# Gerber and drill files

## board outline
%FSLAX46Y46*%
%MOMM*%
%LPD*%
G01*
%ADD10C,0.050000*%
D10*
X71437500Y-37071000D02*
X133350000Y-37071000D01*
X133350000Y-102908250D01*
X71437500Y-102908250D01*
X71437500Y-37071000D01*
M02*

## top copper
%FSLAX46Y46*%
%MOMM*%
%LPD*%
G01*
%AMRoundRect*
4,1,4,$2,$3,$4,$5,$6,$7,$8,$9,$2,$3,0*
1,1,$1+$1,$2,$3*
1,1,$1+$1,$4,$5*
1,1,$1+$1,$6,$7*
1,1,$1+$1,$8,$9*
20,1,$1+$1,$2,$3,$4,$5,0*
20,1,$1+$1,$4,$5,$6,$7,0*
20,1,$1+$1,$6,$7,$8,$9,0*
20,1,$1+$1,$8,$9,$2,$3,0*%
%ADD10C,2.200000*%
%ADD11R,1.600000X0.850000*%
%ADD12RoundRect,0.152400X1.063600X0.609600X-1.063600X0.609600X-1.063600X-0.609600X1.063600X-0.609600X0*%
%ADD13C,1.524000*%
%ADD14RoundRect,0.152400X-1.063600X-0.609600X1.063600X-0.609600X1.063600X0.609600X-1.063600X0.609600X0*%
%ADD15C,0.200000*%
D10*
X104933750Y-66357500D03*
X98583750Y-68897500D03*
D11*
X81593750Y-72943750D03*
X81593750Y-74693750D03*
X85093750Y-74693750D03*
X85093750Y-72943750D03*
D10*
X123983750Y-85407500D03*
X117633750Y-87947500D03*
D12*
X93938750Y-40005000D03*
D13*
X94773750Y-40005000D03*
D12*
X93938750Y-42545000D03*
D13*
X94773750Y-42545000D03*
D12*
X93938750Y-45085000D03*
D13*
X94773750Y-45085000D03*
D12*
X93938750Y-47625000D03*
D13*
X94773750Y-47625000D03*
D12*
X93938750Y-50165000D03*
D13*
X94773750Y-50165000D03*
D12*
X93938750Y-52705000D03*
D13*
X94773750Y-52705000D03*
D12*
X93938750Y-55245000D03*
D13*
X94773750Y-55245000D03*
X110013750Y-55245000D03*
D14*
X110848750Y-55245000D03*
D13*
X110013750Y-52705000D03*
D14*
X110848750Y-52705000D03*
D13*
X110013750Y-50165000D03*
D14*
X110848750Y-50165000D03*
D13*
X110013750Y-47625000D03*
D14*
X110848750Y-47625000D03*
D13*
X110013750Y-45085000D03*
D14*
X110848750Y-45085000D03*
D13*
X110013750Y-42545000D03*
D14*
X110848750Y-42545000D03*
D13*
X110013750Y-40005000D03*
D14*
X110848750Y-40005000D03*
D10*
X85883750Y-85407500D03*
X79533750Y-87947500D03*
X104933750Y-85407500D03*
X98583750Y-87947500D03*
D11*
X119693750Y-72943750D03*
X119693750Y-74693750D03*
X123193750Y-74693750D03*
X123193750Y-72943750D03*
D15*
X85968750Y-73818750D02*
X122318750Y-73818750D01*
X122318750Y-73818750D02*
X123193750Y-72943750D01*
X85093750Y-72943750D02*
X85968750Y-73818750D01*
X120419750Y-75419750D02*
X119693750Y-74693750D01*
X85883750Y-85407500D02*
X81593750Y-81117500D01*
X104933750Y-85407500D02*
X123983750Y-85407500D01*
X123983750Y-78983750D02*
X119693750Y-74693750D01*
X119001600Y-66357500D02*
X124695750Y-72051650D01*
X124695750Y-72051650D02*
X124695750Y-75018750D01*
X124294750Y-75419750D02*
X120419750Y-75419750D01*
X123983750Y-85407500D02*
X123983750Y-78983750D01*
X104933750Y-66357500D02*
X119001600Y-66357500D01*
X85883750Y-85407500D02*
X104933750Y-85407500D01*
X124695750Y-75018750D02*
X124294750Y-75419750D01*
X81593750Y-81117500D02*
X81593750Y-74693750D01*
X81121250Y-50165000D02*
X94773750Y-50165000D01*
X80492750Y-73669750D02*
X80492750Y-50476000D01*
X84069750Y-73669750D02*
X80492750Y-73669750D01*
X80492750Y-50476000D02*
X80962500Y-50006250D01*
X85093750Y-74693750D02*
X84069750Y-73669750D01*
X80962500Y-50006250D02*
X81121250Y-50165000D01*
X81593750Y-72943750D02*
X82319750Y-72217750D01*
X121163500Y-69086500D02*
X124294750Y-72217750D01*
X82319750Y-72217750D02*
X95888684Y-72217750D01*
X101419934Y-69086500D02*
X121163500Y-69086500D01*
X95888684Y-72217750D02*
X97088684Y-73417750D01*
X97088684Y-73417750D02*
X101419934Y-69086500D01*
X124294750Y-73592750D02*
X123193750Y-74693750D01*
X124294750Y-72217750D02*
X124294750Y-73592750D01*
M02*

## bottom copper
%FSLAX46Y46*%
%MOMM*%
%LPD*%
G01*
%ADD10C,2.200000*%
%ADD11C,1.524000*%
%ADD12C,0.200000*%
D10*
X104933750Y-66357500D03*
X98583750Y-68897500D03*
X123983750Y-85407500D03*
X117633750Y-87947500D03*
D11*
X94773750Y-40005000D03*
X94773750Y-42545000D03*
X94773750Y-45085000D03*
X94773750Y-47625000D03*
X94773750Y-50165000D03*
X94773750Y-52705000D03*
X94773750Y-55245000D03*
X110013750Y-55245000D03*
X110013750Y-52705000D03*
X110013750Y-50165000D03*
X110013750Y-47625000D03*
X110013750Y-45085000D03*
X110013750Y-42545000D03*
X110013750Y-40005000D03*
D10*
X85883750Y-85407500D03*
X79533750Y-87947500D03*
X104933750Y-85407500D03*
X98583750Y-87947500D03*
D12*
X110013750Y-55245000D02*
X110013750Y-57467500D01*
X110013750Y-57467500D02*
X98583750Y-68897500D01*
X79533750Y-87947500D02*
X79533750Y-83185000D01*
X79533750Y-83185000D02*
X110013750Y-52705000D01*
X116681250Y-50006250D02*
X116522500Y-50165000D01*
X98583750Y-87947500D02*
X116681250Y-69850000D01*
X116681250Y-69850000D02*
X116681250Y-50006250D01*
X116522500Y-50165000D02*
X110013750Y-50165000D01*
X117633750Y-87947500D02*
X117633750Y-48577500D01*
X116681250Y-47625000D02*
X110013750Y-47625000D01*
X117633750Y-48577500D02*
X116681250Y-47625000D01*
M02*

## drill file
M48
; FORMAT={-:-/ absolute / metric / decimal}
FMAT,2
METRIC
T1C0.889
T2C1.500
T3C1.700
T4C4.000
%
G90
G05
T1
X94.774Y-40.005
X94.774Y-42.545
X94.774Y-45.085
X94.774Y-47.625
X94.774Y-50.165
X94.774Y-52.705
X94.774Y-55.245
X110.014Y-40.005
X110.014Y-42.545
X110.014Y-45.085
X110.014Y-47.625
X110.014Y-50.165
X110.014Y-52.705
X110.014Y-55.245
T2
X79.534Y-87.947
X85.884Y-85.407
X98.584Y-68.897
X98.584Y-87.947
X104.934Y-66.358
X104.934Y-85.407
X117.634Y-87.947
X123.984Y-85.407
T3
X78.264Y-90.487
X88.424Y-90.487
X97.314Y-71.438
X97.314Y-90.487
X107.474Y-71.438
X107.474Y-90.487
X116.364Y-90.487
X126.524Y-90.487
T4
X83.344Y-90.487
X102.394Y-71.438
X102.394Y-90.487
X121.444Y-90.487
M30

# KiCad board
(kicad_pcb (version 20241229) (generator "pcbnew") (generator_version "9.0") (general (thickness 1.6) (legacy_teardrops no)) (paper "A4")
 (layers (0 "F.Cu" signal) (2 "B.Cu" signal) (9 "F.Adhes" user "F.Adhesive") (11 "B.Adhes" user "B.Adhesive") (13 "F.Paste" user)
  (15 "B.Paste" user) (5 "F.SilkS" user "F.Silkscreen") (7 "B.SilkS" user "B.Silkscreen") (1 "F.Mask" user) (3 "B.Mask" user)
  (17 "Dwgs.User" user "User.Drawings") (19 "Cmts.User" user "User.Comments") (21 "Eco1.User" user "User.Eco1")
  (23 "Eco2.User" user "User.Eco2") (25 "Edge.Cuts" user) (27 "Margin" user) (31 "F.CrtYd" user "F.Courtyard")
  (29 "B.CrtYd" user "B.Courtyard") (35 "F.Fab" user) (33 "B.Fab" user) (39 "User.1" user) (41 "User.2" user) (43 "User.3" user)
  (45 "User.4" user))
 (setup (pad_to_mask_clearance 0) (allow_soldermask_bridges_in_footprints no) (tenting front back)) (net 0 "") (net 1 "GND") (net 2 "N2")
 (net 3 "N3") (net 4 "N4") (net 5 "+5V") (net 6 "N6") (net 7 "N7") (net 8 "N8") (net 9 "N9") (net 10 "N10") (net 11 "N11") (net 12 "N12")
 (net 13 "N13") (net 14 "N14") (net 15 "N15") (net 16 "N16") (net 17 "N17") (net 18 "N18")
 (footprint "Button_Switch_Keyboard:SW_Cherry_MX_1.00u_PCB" (layer "F.Cu") (at 104.93375 66.3575)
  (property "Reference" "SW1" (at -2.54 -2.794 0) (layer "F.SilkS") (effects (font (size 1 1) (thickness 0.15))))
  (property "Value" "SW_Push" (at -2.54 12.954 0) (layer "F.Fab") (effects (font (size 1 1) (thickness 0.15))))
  (pad "" np_thru_hole circle (at -7.62 5.08) (size 1.7 1.7) (drill 1.7) (layers "*.Cu" "*.Mask"))
  (pad "" np_thru_hole circle (at -2.54 5.08) (size 4 4) (drill 4) (layers "*.Cu" "*.Mask"))
  (pad "" np_thru_hole circle (at 2.54 5.08) (size 1.7 1.7) (drill 1.7) (layers "*.Cu" "*.Mask"))
  (pad "1" thru_hole circle (at 0 0) (size 2.2 2.2) (drill 1.5) (layers "*.Cu" "*.Mask") (remove_unused_layers no) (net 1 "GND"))
  (pad "2" thru_hole circle (at -6.35 2.54) (size 2.2 2.2) (drill 1.5) (layers "*.Cu" "*.Mask") (remove_unused_layers no) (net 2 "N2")))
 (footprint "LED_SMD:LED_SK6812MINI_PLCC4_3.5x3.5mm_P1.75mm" (layer "F.Cu") (at 83.34375 73.81875)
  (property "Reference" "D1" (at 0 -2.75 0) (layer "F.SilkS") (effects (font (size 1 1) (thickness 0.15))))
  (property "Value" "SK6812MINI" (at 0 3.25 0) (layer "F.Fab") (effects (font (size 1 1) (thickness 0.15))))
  (pad "1" smd rect (at -1.75 -0.875) (size 1.6 0.85) (layers "F.Cu" "F.Mask" "F.Paste") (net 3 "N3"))
  (pad "2" smd rect (at -1.75 0.875) (size 1.6 0.85) (layers "F.Cu" "F.Mask" "F.Paste") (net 1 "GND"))
  (pad "3" smd rect (at 1.75 0.875) (size 1.6 0.85) (layers "F.Cu" "F.Mask" "F.Paste") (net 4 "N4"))
  (pad "4" smd rect (at 1.75 -0.875) (size 1.6 0.85) (layers "F.Cu" "F.Mask" "F.Paste") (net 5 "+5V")))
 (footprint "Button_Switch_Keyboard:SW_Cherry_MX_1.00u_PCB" (layer "F.Cu") (at 123.98375 85.4075)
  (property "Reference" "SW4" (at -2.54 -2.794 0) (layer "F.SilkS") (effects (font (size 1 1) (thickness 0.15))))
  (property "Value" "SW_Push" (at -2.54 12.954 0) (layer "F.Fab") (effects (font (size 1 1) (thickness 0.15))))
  (pad "" np_thru_hole circle (at -7.62 5.08) (size 1.7 1.7) (drill 1.7) (layers "*.Cu" "*.Mask"))
  (pad "" np_thru_hole circle (at -2.54 5.08) (size 4 4) (drill 4) (layers "*.Cu" "*.Mask"))
  (pad "" np_thru_hole circle (at 2.54 5.08) (size 1.7 1.7) (drill 1.7) (layers "*.Cu" "*.Mask"))
  (pad "1" thru_hole circle (at 0 0) (size 2.2 2.2) (drill 1.5) (layers "*.Cu" "*.Mask") (remove_unused_layers no) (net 1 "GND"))
  (pad "2" thru_hole circle (at -6.35 2.54) (size 2.2 2.2) (drill 1.5) (layers "*.Cu" "*.Mask") (remove_unused_layers no) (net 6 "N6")))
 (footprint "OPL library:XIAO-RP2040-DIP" (layer "F.Cu") (at 102.39375 47.625)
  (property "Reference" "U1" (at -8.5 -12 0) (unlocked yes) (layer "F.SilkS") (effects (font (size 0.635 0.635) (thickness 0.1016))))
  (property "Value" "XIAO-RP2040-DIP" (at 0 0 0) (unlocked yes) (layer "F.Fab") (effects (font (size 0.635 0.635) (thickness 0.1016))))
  (pad "1" smd roundrect (at -8.455 -7.62 180) (size 2.432 1.524) (layers "F.Cu" "F.Mask") (roundrect_rratio 0.1) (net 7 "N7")
   (thermal_bridge_angle 45))
  (pad "1" thru_hole circle (at -7.62 -7.62 180) (size 1.524 1.524) (drill 0.889) (layers "*.Cu" "*.Mask") (remove_unused_layers no)
   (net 7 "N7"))
  (pad "2" smd roundrect (at -8.455 -5.08 180) (size 2.432 1.524) (layers "F.Cu" "F.Mask") (roundrect_rratio 0.1) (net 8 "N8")
   (thermal_bridge_angle 45))
  (pad "2" thru_hole circle (at -7.62 -5.08 180) (size 1.524 1.524) (drill 0.889) (layers "*.Cu" "*.Mask") (remove_unused_layers no)
   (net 8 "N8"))
  (pad "3" smd roundrect (at -8.455 -2.54 180) (size 2.432 1.524) (layers "F.Cu" "F.Mask") (roundrect_rratio 0.1) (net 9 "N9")
   (thermal_bridge_angle 45))
  (pad "3" thru_hole circle (at -7.62 -2.54 180) (size 1.524 1.524) (drill 0.889) (layers "*.Cu" "*.Mask") (remove_unused_layers no)
   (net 9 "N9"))
  (pad "4" smd roundrect (at -8.455 0 180) (size 2.432 1.524) (layers "F.Cu" "F.Mask") (roundrect_rratio 0.1) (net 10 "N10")
   (thermal_bridge_angle 45))
  (pad "4" thru_hole circle (at -7.62 0 180) (size 1.524 1.524) (drill 0.889) (layers "*.Cu" "*.Mask") (remove_unused_layers no)
   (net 10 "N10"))
  (pad "5" smd roundrect (at -8.455 2.54 180) (size 2.432 1.524) (layers "F.Cu" "F.Mask") (roundrect_rratio 0.1) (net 4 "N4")
   (thermal_bridge_angle 45))
  (pad "5" thru_hole circle (at -7.62 2.54 180) (size 1.524 1.524) (drill 0.889) (layers "*.Cu" "*.Mask") (remove_unused_layers no)
   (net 4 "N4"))
  (pad "6" smd roundrect (at -8.455 5.08 180) (size 2.432 1.524) (layers "F.Cu" "F.Mask") (roundrect_rratio 0.1) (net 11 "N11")
   (thermal_bridge_angle 45))
  (pad "6" thru_hole circle (at -7.62 5.08 180) (size 1.524 1.524) (drill 0.889) (layers "*.Cu" "*.Mask") (remove_unused_layers no)
   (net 11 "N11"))
  (pad "7" smd roundrect (at -8.455 7.62 180) (size 2.432 1.524) (layers "F.Cu" "F.Mask") (roundrect_rratio 0.1) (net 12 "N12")
   (thermal_bridge_angle 45))
  (pad "7" thru_hole circle (at -7.62 7.62 180) (size 1.524 1.524) (drill 0.889) (layers "*.Cu" "*.Mask") (remove_unused_layers no)
   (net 12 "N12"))
  (pad "8" thru_hole circle (at 7.62 7.62) (size 1.524 1.524) (drill 0.889) (layers "*.Cu" "*.Mask") (remove_unused_layers no) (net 2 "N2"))
  (pad "8" smd roundrect (at 8.455 7.62) (size 2.432 1.524) (layers "F.Cu" "F.Mask") (roundrect_rratio 0.1) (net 2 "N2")
   (thermal_bridge_angle 45))
  (pad "9" thru_hole circle (at 7.62 5.08) (size 1.524 1.524) (drill 0.889) (layers "*.Cu" "*.Mask") (remove_unused_layers no)
   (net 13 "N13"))
  (pad "9" smd roundrect (at 8.455 5.08) (size 2.432 1.524) (layers "F.Cu" "F.Mask") (roundrect_rratio 0.1) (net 13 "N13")
   (thermal_bridge_angle 45))
  (pad "10" thru_hole circle (at 7.62 2.54) (size 1.524 1.524) (drill 0.889) (layers "*.Cu" "*.Mask") (remove_unused_layers no)
   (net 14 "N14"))
  (pad "10" smd roundrect (at 8.455 2.54) (size 2.432 1.524) (layers "F.Cu" "F.Mask") (roundrect_rratio 0.1) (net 14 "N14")
   (thermal_bridge_angle 45))
  (pad "11" thru_hole circle (at 7.62 0) (size 1.524 1.524) (drill 0.889) (layers "*.Cu" "*.Mask") (remove_unused_layers no) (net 6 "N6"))
  (pad "11" smd roundrect (at 8.455 0) (size 2.432 1.524) (layers "F.Cu" "F.Mask") (roundrect_rratio 0.1) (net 6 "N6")
   (thermal_bridge_angle 45))
  (pad "12" thru_hole circle (at 7.62 -2.54) (size 1.524 1.524) (drill 0.889) (layers "*.Cu" "*.Mask") (remove_unused_layers no)
   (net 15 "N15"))
  (pad "12" smd roundrect (at 8.455 -2.54) (size 2.432 1.524) (layers "F.Cu" "F.Mask") (roundrect_rratio 0.1) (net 15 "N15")
   (thermal_bridge_angle 45))
  (pad "13" thru_hole circle (at 7.62 -5.08) (size 1.524 1.524) (drill 0.889) (layers "*.Cu" "*.Mask") (remove_unused_layers no)
   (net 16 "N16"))
  (pad "13" smd roundrect (at 8.455 -5.08) (size 2.432 1.524) (layers "F.Cu" "F.Mask") (roundrect_rratio 0.1) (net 16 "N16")
   (thermal_bridge_angle 45))
  (pad "14" thru_hole circle (at 7.62 -7.62) (size 1.524 1.524) (drill 0.889) (layers "*.Cu" "*.Mask") (remove_unused_layers no)
   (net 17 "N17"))
  (pad "14" smd roundrect (at 8.455 -7.62) (size 2.432 1.524) (layers "F.Cu" "F.Mask") (roundrect_rratio 0.1) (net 17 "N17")
   (thermal_bridge_angle 45)))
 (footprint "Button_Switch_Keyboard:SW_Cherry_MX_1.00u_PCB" (layer "F.Cu") (at 85.88375 85.4075)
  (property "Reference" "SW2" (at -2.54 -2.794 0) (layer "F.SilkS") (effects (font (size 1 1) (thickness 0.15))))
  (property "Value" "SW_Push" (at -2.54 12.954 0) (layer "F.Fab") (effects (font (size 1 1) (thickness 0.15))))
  (pad "" np_thru_hole circle (at -7.62 5.08) (size 1.7 1.7) (drill 1.7) (layers "*.Cu" "*.Mask"))
  (pad "" np_thru_hole circle (at -2.54 5.08) (size 4 4) (drill 4) (layers "*.Cu" "*.Mask"))
  (pad "" np_thru_hole circle (at 2.54 5.08) (size 1.7 1.7) (drill 1.7) (layers "*.Cu" "*.Mask"))
  (pad "1" thru_hole circle (at 0 0) (size 2.2 2.2) (drill 1.5) (layers "*.Cu" "*.Mask") (remove_unused_layers no) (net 1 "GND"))
  (pad "2" thru_hole circle (at -6.35 2.54) (size 2.2 2.2) (drill 1.5) (layers "*.Cu" "*.Mask") (remove_unused_layers no) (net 13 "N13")))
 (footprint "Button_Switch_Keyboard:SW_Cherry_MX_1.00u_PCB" (layer "F.Cu") (at 104.93375 85.4075)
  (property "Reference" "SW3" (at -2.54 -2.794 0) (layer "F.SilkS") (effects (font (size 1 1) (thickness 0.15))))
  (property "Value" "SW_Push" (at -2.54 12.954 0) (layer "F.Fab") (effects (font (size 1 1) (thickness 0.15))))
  (pad "" np_thru_hole circle (at -7.62 5.08) (size 1.7 1.7) (drill 1.7) (layers "*.Cu" "*.Mask"))
  (pad "" np_thru_hole circle (at -2.54 5.08) (size 4 4) (drill 4) (layers "*.Cu" "*.Mask"))
  (pad "" np_thru_hole circle (at 2.54 5.08) (size 1.7 1.7) (drill 1.7) (layers "*.Cu" "*.Mask"))
  (pad "1" thru_hole circle (at 0 0) (size 2.2 2.2) (drill 1.5) (layers "*.Cu" "*.Mask") (remove_unused_layers no) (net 1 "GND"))
  (pad "2" thru_hole circle (at -6.35 2.54) (size 2.2 2.2) (drill 1.5) (layers "*.Cu" "*.Mask") (remove_unused_layers no) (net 14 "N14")))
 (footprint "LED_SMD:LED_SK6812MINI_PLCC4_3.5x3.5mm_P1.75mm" (layer "F.Cu") (at 121.44375 73.81875)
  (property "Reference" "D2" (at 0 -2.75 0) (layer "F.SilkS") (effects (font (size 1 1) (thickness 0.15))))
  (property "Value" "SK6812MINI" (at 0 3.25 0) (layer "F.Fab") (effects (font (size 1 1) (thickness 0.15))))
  (pad "1" smd rect (at -1.75 -0.875) (size 1.6 0.85) (layers "F.Cu" "F.Mask" "F.Paste") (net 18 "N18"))
  (pad "2" smd rect (at -1.75 0.875) (size 1.6 0.85) (layers "F.Cu" "F.Mask" "F.Paste") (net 1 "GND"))
  (pad "3" smd rect (at 1.75 0.875) (size 1.6 0.85) (layers "F.Cu" "F.Mask" "F.Paste") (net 3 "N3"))
  (pad "4" smd rect (at 1.75 -0.875) (size 1.6 0.85) (layers "F.Cu" "F.Mask" "F.Paste") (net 5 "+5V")))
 (gr_rect (start 71.4375 37.071) (end 133.35 102.90825) (stroke (width 0.05) (type default)) (fill no) (layer "Edge.Cuts"))
 (segment (start 85.96875 73.81875) (end 122.31875 73.81875) (width 0.2) (layer "F.Cu") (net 5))
 (segment (start 122.31875 73.81875) (end 123.19375 72.94375) (width 0.2) (layer "F.Cu") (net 5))
 (segment (start 85.09375 72.94375) (end 85.96875 73.81875) (width 0.2) (layer "F.Cu") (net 5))
 (segment (start 120.41975 75.41975) (end 119.69375 74.69375) (width 0.2) (layer "F.Cu") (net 1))
 (segment (start 85.88375 85.4075) (end 81.59375 81.1175) (width 0.2) (layer "F.Cu") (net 1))
 (segment (start 104.93375 85.4075) (end 123.98375 85.4075) (width 0.2) (layer "F.Cu") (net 1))
 (segment (start 123.98375 78.98375) (end 119.69375 74.69375) (width 0.2) (layer "F.Cu") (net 1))
 (segment (start 119.0016 66.3575) (end 124.69575 72.05165) (width 0.2) (layer "F.Cu") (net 1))
 (segment (start 124.69575 72.05165) (end 124.69575 75.01875) (width 0.2) (layer "F.Cu") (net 1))
 (segment (start 124.29475 75.41975) (end 120.41975 75.41975) (width 0.2) (layer "F.Cu") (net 1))
 (segment (start 123.98375 85.4075) (end 123.98375 78.98375) (width 0.2) (layer "F.Cu") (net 1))
 (segment (start 104.93375 66.3575) (end 119.0016 66.3575) (width 0.2) (layer "F.Cu") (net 1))
 (segment (start 85.88375 85.4075) (end 104.93375 85.4075) (width 0.2) (layer "F.Cu") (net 1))
 (segment (start 124.69575 75.01875) (end 124.29475 75.41975) (width 0.2) (layer "F.Cu") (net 1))
 (segment (start 81.59375 81.1175) (end 81.59375 74.69375) (width 0.2) (layer "F.Cu") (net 1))
 (segment (start 81.12125 50.165) (end 94.77375 50.165) (width 0.2) (layer "F.Cu") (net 4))
 (segment (start 80.49275 73.66975) (end 80.49275 50.476) (width 0.2) (layer "F.Cu") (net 4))
 (segment (start 84.06975 73.66975) (end 80.49275 73.66975) (width 0.2) (layer "F.Cu") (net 4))
 (segment (start 80.49275 50.476) (end 80.9625 50.00625) (width 0.2) (layer "F.Cu") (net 4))
 (segment (start 85.09375 74.69375) (end 84.06975 73.66975) (width 0.2) (layer "F.Cu") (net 4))
 (segment (start 80.9625 50.00625) (end 81.12125 50.165) (width 0.2) (layer "F.Cu") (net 4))
 (segment (start 81.59375 72.94375) (end 82.31975 72.21775) (width 0.2) (layer "F.Cu") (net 3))
 (segment (start 121.1635 69.0865) (end 124.29475 72.21775) (width 0.2) (layer "F.Cu") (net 3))
 (segment (start 82.31975 72.21775) (end 95.888684 72.21775) (width 0.2) (layer "F.Cu") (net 3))
 (segment (start 101.419934 69.0865) (end 121.1635 69.0865) (width 0.2) (layer "F.Cu") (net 3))
 (segment (start 95.888684 72.21775) (end 97.088684 73.41775) (width 0.2) (layer "F.Cu") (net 3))
 (segment (start 97.088684 73.41775) (end 101.419934 69.0865) (width 0.2) (layer "F.Cu") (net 3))
 (segment (start 124.29475 73.59275) (end 123.19375 74.69375) (width 0.2) (layer "F.Cu") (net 3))
 (segment (start 124.29475 72.21775) (end 124.29475 73.59275) (width 0.2) (layer "F.Cu") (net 3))
 (segment (start 110.01375 55.245) (end 110.01375 57.4675) (width 0.2) (layer "B.Cu") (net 2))
 (segment (start 110.01375 57.4675) (end 98.58375 68.8975) (width 0.2) (layer "B.Cu") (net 2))
 (segment (start 79.53375 87.9475) (end 79.53375 83.185) (width 0.2) (layer "B.Cu") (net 13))
 (segment (start 79.53375 83.185) (end 110.01375 52.705) (width 0.2) (layer "B.Cu") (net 13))
 (segment (start 116.68125 50.00625) (end 116.5225 50.165) (width 0.2) (layer "B.Cu") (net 14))
 (segment (start 98.58375 87.9475) (end 116.68125 69.85) (width 0.2) (layer "B.Cu") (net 14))
 (segment (start 116.68125 69.85) (end 116.68125 50.00625) (width 0.2) (layer "B.Cu") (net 14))
 (segment (start 116.5225 50.165) (end 110.01375 50.165) (width 0.2) (layer "B.Cu") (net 14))
 (segment (start 117.63375 87.9475) (end 117.63375 48.5775) (width 0.2) (layer "B.Cu") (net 6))
 (segment (start 116.68125 47.625) (end 110.01375 47.625) (width 0.2) (layer "B.Cu") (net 6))
 (segment (start 117.63375 48.5775) (end 116.68125 47.625) (width 0.2) (layer "B.Cu") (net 6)))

